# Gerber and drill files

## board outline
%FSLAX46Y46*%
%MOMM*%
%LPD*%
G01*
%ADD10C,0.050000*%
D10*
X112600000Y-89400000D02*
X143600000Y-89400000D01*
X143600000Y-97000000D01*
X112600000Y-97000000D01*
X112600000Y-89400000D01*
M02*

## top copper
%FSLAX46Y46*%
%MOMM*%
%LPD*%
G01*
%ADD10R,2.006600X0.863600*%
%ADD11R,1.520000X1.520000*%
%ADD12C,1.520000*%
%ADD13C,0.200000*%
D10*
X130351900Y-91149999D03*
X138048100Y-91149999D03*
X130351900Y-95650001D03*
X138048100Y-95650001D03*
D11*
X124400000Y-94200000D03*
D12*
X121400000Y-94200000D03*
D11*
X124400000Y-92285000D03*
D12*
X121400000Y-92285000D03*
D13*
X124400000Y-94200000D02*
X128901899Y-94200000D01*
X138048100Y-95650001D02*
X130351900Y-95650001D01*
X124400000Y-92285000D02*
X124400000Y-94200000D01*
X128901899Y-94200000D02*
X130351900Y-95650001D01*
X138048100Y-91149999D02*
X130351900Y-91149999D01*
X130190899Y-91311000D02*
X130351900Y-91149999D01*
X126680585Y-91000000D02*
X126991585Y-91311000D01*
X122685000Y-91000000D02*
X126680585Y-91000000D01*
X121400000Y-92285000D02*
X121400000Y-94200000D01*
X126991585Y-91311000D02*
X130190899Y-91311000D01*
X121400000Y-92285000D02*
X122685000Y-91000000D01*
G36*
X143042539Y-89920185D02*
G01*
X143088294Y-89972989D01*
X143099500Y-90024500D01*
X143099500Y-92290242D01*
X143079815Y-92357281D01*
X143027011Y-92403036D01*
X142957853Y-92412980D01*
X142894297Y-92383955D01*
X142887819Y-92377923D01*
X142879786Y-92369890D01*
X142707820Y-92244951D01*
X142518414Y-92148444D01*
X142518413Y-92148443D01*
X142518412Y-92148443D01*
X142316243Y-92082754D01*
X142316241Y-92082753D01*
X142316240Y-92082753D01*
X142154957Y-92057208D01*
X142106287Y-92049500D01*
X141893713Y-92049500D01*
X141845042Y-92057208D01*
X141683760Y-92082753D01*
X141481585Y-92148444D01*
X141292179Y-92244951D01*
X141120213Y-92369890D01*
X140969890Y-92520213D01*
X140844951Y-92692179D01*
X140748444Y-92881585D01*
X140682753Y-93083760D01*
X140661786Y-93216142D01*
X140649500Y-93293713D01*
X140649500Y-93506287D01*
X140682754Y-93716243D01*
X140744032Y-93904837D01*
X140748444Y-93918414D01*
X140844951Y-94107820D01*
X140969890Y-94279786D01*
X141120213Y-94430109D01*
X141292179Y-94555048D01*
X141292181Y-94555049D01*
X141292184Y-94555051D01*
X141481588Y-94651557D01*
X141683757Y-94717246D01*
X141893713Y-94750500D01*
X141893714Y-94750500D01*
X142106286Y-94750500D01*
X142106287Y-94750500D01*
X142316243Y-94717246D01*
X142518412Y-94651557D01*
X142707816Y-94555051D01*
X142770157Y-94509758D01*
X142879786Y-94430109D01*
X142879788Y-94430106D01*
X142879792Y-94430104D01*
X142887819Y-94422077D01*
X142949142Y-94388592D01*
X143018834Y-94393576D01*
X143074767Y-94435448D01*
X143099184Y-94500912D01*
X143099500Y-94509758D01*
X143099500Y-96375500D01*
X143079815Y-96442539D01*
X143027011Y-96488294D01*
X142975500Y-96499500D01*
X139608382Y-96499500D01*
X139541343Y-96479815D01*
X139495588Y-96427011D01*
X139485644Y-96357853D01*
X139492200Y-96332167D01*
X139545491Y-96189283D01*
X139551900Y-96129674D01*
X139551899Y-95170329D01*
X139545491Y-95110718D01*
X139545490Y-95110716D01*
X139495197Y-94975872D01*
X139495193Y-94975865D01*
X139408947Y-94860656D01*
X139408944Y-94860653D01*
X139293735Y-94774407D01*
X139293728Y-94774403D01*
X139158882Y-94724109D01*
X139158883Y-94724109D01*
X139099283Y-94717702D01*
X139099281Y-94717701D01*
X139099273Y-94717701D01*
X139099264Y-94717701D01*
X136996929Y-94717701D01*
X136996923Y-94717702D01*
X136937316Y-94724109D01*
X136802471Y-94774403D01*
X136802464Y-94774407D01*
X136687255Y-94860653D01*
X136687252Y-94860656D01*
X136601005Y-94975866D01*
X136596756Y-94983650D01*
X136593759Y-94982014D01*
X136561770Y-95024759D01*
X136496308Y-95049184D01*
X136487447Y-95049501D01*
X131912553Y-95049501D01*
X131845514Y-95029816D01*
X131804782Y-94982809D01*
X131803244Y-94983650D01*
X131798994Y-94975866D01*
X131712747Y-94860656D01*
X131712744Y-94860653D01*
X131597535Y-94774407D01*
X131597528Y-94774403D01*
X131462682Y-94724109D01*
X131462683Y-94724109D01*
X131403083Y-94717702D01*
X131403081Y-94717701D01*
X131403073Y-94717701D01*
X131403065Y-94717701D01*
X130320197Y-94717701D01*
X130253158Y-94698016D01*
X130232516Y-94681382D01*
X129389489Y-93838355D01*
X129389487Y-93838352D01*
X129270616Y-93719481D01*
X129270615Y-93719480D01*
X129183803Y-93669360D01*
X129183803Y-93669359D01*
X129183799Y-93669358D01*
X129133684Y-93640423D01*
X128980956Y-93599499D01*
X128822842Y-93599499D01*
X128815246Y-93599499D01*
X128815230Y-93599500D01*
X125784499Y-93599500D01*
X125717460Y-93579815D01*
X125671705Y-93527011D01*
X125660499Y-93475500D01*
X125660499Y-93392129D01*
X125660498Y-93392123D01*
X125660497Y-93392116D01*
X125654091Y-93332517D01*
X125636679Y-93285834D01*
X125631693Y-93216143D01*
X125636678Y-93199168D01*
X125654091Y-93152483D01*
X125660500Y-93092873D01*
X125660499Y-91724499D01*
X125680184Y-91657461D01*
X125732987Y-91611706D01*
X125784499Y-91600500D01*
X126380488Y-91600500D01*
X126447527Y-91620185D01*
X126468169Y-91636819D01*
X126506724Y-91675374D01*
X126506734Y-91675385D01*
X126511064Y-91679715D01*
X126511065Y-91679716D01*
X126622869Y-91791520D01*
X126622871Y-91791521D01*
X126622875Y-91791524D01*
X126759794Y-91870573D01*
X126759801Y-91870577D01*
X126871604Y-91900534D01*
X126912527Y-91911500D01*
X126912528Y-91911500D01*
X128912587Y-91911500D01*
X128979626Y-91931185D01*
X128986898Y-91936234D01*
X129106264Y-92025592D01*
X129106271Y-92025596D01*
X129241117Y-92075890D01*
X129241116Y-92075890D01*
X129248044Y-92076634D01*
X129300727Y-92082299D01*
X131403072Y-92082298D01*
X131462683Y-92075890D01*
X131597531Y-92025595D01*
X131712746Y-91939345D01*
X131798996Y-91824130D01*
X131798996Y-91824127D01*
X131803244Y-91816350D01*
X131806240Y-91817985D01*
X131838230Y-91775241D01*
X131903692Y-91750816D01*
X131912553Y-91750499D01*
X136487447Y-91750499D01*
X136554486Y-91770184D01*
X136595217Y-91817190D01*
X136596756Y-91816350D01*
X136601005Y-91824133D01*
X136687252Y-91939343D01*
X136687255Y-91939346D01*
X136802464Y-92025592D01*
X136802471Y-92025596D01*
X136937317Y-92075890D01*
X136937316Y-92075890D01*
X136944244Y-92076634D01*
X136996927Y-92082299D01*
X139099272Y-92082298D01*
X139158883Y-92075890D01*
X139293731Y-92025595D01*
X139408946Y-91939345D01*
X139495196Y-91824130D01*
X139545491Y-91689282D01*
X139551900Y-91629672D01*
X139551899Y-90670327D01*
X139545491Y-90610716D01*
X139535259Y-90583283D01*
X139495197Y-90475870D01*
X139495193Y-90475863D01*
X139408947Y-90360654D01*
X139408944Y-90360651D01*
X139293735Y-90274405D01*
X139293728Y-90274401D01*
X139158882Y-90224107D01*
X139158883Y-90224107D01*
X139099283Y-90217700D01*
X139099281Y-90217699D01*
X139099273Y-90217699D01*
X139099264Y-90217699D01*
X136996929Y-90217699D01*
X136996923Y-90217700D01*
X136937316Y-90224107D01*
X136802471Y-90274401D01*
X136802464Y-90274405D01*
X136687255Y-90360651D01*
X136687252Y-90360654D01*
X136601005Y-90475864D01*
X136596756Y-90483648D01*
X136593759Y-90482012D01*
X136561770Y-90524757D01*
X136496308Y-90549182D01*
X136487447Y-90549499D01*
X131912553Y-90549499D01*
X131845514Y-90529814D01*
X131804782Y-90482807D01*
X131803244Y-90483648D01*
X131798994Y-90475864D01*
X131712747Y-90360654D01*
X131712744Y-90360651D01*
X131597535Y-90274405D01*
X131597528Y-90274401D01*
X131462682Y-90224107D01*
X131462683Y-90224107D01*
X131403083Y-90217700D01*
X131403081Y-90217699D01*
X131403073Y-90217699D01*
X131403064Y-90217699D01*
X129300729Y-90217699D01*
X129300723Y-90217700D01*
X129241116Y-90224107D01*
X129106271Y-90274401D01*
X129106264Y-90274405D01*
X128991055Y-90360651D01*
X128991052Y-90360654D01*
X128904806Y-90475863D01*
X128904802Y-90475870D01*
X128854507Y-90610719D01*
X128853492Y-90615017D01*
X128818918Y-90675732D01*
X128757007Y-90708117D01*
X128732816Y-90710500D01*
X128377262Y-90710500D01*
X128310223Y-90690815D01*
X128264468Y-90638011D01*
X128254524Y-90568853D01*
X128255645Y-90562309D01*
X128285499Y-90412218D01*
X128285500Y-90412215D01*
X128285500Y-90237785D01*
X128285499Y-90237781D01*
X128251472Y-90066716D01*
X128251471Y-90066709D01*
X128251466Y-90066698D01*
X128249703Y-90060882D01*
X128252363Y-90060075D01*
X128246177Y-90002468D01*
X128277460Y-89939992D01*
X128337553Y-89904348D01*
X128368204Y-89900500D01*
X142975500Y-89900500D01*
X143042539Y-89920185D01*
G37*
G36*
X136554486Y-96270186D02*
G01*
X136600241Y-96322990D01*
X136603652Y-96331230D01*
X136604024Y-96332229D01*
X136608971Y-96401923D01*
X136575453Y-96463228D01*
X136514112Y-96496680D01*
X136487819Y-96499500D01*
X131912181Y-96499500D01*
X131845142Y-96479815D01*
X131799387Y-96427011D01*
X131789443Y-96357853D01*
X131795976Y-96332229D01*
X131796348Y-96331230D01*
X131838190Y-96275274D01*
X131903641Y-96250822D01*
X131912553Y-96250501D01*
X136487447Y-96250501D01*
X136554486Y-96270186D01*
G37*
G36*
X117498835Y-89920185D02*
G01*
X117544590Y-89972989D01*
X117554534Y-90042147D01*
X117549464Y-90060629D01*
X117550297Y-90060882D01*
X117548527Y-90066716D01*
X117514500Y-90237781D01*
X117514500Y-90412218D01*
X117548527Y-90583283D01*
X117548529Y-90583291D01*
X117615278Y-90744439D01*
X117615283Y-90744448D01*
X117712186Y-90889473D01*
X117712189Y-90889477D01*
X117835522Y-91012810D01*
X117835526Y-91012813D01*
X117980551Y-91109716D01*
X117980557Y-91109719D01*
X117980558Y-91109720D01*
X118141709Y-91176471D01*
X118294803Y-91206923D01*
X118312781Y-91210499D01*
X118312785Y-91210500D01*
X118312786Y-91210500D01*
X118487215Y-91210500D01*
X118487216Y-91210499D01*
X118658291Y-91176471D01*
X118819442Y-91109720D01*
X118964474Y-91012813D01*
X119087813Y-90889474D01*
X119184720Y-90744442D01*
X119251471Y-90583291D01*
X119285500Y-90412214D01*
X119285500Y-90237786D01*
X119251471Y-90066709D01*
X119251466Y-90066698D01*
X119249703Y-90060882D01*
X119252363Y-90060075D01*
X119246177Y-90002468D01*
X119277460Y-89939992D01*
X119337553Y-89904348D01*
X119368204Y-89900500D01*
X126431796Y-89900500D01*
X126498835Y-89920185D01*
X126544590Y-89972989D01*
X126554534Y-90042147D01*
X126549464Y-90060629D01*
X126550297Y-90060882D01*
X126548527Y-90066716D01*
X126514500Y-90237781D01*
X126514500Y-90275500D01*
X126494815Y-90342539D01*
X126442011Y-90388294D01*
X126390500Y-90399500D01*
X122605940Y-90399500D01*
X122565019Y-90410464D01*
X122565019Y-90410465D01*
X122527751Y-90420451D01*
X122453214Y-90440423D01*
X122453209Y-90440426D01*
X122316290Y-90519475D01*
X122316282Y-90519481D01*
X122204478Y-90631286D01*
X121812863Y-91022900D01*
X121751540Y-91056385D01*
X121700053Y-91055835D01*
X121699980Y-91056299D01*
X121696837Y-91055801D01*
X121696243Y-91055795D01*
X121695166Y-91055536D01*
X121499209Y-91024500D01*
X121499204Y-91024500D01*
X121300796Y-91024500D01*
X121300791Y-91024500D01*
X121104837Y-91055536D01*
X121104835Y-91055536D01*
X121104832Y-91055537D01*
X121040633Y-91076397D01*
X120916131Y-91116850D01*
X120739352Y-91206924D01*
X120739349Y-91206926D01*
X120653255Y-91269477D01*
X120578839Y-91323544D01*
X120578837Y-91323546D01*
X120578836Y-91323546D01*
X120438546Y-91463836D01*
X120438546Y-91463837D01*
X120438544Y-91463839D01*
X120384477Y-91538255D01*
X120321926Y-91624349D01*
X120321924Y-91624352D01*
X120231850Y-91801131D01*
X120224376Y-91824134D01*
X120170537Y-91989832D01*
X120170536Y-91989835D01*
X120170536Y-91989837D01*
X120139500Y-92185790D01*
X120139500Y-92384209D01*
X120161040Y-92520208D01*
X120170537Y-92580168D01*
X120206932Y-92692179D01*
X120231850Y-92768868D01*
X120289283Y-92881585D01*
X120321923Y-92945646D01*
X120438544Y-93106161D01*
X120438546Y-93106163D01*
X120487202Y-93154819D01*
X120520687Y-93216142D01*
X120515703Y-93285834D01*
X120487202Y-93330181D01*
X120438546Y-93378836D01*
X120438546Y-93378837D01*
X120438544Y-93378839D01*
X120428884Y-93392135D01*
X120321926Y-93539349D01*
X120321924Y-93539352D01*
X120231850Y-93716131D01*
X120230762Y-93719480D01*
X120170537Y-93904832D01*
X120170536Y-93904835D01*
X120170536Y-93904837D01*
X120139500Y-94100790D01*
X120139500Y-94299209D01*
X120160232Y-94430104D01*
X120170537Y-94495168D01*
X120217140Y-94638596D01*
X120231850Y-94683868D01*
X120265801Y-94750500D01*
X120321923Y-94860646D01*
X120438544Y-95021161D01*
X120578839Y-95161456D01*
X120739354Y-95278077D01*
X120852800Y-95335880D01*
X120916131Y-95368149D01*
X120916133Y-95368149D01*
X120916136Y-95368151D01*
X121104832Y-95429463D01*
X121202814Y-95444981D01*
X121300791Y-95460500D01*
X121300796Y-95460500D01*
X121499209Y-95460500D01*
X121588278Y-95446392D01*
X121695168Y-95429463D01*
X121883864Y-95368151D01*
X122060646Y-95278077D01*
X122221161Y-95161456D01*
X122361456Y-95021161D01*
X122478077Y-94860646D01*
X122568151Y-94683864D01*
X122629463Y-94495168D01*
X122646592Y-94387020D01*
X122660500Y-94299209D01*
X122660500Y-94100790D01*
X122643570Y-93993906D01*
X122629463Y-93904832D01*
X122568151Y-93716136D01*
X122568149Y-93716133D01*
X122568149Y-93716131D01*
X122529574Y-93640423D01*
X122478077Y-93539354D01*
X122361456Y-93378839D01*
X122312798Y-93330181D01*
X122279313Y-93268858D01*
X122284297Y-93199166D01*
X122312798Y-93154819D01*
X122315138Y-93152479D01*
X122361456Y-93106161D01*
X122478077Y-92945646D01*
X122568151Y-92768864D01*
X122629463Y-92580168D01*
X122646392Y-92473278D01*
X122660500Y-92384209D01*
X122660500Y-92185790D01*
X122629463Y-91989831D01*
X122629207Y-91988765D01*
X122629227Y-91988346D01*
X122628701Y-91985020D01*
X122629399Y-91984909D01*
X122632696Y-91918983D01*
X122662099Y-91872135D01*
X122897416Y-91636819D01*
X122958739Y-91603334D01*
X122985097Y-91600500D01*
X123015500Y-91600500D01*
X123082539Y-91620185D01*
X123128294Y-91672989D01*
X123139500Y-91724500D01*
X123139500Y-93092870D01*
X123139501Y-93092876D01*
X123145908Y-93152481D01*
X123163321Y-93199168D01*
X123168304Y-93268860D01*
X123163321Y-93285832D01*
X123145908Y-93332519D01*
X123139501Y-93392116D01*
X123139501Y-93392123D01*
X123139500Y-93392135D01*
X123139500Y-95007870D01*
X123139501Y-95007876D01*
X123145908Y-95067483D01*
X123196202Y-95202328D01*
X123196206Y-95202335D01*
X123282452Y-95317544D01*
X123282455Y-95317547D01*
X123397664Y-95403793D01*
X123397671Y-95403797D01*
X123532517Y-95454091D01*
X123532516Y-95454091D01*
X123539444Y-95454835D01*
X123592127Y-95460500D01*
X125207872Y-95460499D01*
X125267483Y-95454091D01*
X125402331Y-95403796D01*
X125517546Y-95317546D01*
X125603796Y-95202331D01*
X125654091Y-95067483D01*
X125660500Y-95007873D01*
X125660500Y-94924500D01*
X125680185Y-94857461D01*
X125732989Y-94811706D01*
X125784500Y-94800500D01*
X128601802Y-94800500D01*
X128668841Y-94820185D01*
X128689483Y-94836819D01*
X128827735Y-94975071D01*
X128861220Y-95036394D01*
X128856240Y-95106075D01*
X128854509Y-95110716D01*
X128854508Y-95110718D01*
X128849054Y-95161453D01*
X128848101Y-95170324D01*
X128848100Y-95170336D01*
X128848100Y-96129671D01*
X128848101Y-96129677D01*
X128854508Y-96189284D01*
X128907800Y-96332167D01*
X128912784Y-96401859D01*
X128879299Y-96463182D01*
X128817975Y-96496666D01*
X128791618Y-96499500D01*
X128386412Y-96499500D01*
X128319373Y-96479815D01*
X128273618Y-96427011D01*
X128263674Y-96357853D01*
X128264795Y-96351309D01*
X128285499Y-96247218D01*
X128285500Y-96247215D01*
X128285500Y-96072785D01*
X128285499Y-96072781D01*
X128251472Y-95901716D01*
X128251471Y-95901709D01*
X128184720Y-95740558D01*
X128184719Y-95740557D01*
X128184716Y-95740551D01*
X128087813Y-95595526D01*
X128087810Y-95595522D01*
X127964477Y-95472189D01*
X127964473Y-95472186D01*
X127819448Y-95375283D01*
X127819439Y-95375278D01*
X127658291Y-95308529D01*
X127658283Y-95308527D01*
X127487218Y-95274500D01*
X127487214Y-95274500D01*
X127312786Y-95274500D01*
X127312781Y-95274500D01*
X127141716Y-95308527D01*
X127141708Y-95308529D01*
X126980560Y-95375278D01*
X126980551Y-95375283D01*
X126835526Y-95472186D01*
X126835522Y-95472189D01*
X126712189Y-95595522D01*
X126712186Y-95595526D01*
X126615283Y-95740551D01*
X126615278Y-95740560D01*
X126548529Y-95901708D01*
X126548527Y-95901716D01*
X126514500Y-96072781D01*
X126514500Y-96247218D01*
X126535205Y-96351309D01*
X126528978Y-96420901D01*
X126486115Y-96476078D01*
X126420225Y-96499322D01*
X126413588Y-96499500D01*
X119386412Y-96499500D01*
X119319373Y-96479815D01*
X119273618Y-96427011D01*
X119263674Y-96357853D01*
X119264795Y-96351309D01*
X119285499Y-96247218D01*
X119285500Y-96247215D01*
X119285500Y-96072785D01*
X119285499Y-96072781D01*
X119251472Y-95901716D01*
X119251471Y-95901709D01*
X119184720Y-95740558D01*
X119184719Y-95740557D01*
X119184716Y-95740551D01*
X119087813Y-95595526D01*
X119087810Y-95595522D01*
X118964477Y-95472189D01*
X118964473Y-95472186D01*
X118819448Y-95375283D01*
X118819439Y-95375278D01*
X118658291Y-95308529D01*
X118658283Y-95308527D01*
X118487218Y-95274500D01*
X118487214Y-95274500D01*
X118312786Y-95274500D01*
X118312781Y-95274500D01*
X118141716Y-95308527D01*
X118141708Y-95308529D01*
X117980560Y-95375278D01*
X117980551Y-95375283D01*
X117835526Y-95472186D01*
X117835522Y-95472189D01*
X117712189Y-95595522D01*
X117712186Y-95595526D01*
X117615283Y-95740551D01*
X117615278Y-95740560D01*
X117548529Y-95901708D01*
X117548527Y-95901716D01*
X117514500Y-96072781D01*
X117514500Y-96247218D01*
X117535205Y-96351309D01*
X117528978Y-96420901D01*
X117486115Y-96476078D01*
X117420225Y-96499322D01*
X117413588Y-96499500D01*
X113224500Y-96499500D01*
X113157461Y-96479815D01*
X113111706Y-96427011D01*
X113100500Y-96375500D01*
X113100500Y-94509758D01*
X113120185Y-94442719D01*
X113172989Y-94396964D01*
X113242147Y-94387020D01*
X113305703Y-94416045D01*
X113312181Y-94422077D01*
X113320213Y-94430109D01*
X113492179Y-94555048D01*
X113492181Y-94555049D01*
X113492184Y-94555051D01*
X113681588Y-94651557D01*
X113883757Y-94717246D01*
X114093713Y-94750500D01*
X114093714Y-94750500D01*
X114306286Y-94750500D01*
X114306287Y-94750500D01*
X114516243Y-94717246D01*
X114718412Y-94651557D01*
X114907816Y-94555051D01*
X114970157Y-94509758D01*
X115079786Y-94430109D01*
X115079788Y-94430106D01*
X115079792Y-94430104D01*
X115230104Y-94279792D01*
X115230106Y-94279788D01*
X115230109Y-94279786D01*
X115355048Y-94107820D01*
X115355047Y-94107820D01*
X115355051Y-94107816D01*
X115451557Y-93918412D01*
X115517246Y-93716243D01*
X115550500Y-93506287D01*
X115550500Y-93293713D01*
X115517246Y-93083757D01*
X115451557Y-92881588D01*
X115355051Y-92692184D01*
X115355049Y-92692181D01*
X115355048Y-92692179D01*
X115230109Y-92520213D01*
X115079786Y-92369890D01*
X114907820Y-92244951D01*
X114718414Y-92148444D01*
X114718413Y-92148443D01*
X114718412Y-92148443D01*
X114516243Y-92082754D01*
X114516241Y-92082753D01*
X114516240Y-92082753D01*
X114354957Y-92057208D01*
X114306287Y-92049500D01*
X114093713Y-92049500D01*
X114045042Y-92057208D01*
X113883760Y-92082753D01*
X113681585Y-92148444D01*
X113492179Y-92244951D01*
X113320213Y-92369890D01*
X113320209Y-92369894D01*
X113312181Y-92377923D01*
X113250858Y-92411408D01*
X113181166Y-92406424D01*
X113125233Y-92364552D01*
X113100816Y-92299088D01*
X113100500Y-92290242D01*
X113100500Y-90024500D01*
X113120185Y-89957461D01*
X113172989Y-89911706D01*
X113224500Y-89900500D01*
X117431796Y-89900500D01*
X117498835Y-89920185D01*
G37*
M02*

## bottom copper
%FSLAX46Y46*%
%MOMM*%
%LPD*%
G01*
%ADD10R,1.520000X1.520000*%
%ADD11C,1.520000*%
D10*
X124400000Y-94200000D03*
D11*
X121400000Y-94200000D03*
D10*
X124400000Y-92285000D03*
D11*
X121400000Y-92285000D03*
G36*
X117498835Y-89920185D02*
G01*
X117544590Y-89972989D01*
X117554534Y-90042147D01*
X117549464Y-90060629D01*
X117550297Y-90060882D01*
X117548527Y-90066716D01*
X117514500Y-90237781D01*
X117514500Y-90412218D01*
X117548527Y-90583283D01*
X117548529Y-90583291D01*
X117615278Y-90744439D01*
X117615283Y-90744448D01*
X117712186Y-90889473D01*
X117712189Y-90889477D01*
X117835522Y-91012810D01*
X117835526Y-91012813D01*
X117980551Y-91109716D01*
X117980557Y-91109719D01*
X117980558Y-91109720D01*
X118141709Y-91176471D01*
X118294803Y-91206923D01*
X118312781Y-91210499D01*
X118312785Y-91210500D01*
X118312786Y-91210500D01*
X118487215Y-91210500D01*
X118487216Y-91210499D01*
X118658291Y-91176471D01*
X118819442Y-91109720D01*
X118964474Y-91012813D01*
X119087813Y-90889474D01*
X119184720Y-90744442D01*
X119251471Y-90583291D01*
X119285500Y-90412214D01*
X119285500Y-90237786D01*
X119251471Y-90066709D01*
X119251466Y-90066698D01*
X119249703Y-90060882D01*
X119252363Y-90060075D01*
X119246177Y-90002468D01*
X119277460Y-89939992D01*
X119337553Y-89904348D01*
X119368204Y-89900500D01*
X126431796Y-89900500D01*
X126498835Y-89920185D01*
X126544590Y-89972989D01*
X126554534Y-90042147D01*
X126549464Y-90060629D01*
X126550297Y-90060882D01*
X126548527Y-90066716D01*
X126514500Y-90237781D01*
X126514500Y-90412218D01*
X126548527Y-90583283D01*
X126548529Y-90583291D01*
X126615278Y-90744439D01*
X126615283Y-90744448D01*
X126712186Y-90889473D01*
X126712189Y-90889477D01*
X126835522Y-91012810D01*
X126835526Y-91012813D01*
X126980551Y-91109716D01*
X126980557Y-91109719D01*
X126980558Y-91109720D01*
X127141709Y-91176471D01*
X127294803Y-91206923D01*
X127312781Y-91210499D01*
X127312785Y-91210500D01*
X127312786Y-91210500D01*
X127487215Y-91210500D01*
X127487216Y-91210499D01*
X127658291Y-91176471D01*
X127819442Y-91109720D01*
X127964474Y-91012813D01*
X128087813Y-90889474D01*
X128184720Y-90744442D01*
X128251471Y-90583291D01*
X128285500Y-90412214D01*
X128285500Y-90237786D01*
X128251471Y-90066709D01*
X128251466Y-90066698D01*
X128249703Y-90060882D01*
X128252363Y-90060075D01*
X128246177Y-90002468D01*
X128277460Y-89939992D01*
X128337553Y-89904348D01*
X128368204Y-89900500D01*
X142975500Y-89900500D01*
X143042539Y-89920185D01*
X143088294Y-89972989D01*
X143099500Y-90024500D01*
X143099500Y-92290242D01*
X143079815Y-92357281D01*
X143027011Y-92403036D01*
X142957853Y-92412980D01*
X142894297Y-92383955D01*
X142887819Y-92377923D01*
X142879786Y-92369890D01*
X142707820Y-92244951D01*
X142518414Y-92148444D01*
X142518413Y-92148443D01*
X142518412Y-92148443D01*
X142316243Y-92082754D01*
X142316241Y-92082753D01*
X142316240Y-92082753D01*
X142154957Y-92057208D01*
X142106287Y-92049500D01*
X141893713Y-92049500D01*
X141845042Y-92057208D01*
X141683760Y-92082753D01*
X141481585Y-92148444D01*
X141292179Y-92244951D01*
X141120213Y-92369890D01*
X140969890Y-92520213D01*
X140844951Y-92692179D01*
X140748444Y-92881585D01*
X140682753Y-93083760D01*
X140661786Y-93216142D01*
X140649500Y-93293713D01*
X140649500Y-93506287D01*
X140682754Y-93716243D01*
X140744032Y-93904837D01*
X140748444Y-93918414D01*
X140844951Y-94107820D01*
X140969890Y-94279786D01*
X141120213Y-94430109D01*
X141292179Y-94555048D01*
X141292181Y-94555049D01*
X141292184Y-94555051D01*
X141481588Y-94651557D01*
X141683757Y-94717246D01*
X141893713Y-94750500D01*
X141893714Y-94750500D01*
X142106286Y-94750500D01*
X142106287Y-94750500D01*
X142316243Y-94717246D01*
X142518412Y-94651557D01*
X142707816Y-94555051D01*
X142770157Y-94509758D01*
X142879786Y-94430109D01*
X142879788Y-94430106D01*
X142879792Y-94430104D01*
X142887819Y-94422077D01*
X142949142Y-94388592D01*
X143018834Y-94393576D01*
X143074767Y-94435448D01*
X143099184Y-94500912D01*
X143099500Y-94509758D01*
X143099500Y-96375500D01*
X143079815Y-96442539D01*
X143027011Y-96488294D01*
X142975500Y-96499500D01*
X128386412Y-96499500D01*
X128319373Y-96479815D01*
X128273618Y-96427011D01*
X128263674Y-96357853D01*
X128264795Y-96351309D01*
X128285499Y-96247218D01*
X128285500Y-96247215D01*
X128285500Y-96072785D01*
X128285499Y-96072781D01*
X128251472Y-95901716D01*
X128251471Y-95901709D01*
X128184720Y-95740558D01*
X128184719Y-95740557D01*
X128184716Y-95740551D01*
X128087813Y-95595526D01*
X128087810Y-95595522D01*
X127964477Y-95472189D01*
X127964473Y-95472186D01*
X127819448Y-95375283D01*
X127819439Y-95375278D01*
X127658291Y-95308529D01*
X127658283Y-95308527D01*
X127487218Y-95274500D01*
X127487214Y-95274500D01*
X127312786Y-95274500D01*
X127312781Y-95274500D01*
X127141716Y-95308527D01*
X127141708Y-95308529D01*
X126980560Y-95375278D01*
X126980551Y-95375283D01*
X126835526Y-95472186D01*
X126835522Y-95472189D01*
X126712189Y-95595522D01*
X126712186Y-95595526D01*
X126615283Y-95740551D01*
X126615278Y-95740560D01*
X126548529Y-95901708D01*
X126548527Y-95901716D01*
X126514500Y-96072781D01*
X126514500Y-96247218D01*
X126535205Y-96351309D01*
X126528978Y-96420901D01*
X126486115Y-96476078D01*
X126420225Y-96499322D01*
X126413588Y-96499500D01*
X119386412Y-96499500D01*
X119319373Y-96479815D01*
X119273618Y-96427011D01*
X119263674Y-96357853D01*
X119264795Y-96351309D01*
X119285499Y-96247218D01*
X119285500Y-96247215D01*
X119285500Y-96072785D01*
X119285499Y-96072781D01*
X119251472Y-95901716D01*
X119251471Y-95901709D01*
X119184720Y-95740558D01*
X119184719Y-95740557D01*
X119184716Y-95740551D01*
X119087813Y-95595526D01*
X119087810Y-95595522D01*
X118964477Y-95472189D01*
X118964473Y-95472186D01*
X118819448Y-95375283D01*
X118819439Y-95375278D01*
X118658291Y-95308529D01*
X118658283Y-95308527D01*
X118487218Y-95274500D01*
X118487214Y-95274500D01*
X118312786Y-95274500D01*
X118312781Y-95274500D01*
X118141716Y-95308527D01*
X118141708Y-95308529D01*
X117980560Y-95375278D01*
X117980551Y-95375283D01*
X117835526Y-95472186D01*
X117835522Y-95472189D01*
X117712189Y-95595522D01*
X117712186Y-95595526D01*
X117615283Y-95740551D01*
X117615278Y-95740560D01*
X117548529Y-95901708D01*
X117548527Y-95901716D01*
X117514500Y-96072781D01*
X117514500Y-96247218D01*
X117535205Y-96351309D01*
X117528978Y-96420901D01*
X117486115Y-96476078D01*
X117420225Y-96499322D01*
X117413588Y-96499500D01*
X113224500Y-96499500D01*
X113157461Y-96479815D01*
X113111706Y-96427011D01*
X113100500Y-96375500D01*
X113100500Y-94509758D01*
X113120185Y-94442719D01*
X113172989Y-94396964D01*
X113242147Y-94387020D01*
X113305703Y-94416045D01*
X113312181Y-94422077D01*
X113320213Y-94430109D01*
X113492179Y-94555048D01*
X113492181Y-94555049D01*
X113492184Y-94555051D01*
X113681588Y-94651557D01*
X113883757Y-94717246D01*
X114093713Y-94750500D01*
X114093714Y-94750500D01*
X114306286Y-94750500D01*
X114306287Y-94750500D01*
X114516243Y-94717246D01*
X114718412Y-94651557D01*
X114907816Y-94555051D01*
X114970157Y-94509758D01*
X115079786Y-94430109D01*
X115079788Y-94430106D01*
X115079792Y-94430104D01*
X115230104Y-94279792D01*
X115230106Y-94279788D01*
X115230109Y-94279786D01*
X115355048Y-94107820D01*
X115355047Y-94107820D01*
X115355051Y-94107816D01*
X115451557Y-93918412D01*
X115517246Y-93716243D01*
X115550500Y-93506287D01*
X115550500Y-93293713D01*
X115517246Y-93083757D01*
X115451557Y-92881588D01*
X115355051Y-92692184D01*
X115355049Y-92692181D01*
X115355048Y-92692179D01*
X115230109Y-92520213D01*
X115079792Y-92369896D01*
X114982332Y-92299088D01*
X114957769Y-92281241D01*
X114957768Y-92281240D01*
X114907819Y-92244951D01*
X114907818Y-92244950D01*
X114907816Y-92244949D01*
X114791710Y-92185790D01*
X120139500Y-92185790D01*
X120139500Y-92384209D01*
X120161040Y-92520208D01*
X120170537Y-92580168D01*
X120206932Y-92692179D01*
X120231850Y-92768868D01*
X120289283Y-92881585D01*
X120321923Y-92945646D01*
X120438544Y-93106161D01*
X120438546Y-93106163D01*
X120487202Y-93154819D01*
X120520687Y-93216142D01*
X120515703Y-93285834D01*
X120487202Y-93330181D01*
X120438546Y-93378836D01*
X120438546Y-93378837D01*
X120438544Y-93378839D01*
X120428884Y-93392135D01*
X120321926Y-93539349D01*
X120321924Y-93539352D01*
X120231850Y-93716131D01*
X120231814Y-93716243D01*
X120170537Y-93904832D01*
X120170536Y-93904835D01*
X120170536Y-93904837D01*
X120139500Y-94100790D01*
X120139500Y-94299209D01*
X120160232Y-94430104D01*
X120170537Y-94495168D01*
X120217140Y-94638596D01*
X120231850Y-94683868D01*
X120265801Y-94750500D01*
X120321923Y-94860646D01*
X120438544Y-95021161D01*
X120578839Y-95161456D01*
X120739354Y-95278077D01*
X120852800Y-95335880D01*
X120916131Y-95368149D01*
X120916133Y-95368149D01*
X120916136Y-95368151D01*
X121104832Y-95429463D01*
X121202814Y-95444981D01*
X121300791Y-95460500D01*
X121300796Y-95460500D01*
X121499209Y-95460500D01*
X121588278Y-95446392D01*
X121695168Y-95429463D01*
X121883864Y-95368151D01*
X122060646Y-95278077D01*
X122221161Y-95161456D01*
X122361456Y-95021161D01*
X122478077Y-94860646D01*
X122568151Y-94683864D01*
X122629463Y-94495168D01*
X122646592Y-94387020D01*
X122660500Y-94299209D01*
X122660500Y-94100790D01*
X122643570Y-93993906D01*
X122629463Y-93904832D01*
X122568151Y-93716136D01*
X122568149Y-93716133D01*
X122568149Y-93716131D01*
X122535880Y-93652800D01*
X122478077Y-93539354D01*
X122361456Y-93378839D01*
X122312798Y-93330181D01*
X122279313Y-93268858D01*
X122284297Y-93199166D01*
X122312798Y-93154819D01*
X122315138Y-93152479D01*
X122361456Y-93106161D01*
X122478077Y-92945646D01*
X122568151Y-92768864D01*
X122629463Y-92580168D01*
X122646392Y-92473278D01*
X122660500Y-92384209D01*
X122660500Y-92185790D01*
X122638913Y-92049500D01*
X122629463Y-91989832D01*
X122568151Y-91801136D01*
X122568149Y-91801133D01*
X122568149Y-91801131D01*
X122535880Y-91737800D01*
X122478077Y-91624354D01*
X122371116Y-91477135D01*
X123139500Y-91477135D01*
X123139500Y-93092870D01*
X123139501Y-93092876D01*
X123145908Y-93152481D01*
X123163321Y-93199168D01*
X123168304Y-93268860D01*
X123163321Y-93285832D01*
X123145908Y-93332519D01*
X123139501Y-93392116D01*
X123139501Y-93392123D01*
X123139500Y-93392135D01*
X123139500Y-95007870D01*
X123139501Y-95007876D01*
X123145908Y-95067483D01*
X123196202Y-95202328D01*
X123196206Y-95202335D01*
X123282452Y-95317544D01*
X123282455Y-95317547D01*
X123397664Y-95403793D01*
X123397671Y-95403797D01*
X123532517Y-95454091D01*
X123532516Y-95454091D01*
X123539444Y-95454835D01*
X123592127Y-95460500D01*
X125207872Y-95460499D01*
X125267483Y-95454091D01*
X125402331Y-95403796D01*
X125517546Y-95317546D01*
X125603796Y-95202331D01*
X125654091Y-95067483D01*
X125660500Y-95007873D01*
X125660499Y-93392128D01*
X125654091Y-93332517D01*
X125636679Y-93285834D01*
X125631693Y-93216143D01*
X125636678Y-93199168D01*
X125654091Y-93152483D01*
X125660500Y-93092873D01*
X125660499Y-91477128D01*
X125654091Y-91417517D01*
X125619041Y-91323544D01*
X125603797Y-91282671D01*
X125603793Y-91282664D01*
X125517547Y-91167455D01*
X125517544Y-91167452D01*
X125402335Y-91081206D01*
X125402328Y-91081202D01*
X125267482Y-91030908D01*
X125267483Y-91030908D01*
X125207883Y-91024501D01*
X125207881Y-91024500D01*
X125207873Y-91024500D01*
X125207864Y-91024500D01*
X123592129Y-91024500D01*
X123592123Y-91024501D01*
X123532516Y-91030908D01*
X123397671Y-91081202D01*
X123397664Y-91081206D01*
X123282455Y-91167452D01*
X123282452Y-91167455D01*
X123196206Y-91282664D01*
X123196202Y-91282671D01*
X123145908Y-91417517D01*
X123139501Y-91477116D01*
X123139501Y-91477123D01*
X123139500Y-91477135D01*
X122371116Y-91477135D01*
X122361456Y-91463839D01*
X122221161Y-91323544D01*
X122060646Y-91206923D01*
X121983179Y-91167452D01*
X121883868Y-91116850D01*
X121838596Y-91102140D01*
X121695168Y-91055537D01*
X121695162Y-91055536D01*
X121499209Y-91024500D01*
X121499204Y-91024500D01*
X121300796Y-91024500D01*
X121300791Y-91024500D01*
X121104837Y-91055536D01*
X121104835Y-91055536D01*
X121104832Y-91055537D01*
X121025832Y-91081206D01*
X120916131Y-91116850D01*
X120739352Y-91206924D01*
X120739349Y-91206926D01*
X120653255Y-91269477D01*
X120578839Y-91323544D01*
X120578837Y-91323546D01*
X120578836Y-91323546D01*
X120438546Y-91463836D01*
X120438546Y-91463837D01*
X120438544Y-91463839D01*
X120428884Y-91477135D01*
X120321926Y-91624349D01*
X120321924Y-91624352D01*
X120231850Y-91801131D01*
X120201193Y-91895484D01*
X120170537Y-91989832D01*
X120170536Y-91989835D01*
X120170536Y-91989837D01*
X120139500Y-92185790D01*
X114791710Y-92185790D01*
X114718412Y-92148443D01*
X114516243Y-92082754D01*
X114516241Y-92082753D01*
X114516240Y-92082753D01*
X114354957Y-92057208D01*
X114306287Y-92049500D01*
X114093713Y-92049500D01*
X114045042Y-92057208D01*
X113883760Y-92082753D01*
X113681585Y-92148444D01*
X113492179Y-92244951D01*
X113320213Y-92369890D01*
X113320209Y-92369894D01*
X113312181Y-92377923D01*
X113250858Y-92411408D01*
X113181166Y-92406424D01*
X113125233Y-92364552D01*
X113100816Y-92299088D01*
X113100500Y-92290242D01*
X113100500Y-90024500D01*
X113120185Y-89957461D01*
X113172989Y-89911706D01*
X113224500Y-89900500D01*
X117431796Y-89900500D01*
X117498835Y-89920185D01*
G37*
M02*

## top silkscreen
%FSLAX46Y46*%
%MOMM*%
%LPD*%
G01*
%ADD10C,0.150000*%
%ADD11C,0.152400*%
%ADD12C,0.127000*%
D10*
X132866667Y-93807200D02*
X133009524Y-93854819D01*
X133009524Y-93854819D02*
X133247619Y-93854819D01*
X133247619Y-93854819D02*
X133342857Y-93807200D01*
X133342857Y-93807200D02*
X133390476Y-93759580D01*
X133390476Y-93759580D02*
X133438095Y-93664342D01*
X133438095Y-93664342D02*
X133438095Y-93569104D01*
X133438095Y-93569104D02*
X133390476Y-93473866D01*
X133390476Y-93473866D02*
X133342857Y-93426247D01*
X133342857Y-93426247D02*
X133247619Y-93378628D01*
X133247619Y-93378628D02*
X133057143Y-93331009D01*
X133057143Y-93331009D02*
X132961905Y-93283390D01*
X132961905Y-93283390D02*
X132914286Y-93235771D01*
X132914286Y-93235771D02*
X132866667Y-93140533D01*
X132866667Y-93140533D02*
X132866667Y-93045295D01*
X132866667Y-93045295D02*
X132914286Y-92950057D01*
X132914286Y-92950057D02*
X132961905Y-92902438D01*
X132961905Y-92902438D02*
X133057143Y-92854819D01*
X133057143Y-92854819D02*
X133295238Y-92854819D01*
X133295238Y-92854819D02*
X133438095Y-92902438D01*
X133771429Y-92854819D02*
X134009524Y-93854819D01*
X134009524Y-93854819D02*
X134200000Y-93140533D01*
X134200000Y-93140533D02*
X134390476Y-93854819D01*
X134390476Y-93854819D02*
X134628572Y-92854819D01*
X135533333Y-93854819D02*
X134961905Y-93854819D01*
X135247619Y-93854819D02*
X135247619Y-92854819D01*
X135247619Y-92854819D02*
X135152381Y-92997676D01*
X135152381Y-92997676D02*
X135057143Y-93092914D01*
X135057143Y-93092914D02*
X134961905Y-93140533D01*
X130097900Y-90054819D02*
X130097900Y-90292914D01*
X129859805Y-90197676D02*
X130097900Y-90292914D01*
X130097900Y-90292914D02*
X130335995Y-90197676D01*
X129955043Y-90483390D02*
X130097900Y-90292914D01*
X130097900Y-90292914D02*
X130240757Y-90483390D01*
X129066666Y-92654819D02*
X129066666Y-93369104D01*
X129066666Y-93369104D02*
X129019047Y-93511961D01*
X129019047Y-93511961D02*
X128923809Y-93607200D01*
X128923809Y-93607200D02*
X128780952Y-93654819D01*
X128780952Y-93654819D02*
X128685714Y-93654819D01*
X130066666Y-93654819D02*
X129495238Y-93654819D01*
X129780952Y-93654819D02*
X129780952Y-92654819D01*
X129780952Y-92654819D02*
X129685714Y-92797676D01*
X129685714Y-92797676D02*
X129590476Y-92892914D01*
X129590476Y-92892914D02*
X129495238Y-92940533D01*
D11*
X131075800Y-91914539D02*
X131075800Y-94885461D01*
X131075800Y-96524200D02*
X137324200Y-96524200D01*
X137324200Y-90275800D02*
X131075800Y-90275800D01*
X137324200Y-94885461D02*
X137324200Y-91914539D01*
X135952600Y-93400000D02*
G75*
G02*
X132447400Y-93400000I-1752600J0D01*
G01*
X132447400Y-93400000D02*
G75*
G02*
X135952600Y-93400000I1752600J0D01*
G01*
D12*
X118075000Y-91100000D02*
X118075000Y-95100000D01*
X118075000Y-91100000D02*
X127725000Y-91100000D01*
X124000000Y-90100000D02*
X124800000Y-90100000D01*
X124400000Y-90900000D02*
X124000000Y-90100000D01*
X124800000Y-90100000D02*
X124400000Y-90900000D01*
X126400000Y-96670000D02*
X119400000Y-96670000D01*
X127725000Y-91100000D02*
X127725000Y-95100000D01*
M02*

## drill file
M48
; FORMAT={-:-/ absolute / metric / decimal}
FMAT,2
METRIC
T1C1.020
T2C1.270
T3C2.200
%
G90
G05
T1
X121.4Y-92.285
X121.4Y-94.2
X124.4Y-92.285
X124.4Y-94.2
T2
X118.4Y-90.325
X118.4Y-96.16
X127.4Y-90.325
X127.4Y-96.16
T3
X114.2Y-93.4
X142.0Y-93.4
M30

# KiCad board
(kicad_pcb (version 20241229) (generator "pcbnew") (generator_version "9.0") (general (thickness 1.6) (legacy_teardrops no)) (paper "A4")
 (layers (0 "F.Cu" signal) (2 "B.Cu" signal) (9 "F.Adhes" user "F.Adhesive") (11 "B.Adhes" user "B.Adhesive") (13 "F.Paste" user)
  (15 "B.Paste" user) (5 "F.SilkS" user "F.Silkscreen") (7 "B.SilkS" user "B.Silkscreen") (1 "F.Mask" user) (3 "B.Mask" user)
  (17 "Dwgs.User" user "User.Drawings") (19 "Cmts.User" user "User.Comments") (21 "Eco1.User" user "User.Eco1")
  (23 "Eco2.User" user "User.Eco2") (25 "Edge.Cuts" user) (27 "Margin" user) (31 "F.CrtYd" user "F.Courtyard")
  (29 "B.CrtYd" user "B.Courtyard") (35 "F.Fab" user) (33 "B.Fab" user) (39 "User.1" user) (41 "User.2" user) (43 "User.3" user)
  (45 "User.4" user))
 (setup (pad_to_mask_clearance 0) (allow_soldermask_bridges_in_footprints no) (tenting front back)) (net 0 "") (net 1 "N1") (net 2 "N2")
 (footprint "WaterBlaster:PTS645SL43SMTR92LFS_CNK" (layer "F.Cu") (at 134.2 93.4)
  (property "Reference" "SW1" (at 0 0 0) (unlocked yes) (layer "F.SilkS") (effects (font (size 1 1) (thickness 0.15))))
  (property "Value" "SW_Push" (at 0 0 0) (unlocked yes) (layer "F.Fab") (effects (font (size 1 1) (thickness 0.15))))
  (fp_line (start -3.1242 -1.485461) (end -3.1242 1.485461) (stroke (width 0.1524) (type solid)) (layer "F.SilkS"))
  (fp_line (start -3.1242 3.1242) (end 3.1242 3.1242) (stroke (width 0.1524) (type solid)) (layer "F.SilkS"))
  (fp_line (start 3.1242 -3.1242) (end -3.1242 -3.1242) (stroke (width 0.1524) (type solid)) (layer "F.SilkS"))
  (fp_line (start 3.1242 1.485461) (end 3.1242 -1.485461) (stroke (width 0.1524) (type solid)) (layer "F.SilkS"))
  (fp_circle (center 0 0) (end 1.7526 0) (stroke (width 0.1524) (type solid)) (fill no) (layer "F.SilkS"))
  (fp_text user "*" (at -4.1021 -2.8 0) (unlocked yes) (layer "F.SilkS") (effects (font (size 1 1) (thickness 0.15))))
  (pad "1" smd rect (at -3.8481 -2.250001) (size 2.0066 0.8636) (layers "F.Cu" "F.Mask" "F.Paste") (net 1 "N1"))
  (pad "1" smd rect (at 3.8481 -2.250001) (size 2.0066 0.8636) (layers "F.Cu" "F.Mask" "F.Paste") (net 1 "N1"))
  (pad "2" smd rect (at -3.8481 2.250001) (size 2.0066 0.8636) (layers "F.Cu" "F.Mask" "F.Paste") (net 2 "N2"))
  (pad "2" smd rect (at 3.8481 2.250001) (size 2.0066 0.8636) (layers "F.Cu" "F.Mask" "F.Paste") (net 2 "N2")))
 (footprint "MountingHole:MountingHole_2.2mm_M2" (layer "F.Cu") (at 142 93.4)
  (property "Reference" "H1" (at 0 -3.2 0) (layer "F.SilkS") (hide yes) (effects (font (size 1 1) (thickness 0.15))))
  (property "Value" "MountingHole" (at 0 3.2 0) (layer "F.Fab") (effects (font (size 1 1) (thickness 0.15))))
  (pad "" np_thru_hole circle (at 0 0) (size 2.2 2.2) (drill 2.2) (layers "*.Cu" "*.Mask")))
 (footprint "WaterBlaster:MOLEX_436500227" (layer "F.Cu") (at 124.4 94.2)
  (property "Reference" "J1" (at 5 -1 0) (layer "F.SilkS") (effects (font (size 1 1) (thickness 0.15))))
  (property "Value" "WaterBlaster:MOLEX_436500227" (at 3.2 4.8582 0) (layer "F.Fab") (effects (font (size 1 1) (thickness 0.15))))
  (fp_line (start -6.325 -3.1) (end -6.325 0.9) (stroke (width 0.127) (type solid)) (layer "F.SilkS"))
  (fp_line (start -6.325 -3.1) (end 3.325 -3.1) (stroke (width 0.127) (type solid)) (layer "F.SilkS"))
  (fp_line (start -0.4 -4.1) (end 0.4 -4.1) (stroke (width 0.127) (type solid)) (layer "F.SilkS"))
  (fp_line (start 0 -3.3) (end -0.4 -4.1) (stroke (width 0.127) (type solid)) (layer "F.SilkS"))
  (fp_line (start 0.4 -4.1) (end 0 -3.3) (stroke (width 0.127) (type solid)) (layer "F.SilkS"))
  (fp_line (start 2 2.47) (end -5 2.47) (stroke (width 0.127) (type solid)) (layer "F.SilkS"))
  (fp_line (start 3.325 -3.1) (end 3.325 0.9) (stroke (width 0.127) (type solid)) (layer "F.SilkS"))
  (pad "" np_thru_hole circle (at -6 1.96) (size 1.27 1.27) (drill 1.27) (layers "*.Cu" "*.Mask"))
  (pad "" np_thru_hole circle (at 3 1.96) (size 1.27 1.27) (drill 1.27) (layers "*.Cu" "*.Mask"))
  (pad "1" thru_hole rect (at 0 0) (size 1.52 1.52) (drill 1.02) (layers "*.Cu") (remove_unused_layers no) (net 2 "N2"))
  (pad "2" thru_hole circle (at -3 0) (size 1.52 1.52) (drill 1.02) (layers "*.Cu") (remove_unused_layers no) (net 1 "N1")))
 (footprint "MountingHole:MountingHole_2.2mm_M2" (layer "F.Cu") (at 114.2 93.4)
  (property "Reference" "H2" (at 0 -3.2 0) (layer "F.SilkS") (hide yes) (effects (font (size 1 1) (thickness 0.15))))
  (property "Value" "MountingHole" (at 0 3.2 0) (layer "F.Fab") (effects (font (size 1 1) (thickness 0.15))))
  (pad "" np_thru_hole circle (at 0 0) (size 2.2 2.2) (drill 2.2) (layers "*.Cu" "*.Mask")))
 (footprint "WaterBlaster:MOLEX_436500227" (layer "B.Cu") (at 124.4 92.285)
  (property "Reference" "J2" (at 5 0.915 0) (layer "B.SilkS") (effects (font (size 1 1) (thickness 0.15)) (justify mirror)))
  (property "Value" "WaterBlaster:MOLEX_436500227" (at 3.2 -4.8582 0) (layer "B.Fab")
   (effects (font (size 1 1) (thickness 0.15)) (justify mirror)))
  (pad "" np_thru_hole circle (at -6 -1.96) (size 1.27 1.27) (drill 1.27) (layers "*.Cu" "*.Mask"))
  (pad "" np_thru_hole circle (at 3 -1.96) (size 1.27 1.27) (drill 1.27) (layers "*.Cu" "*.Mask"))
  (pad "1" thru_hole rect (at 0 0) (size 1.52 1.52) (drill 1.02) (layers "*.Cu") (remove_unused_layers no) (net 2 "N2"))
  (pad "2" thru_hole circle (at -3 0) (size 1.52 1.52) (drill 1.02) (layers "*.Cu") (remove_unused_layers no) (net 1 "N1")))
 (gr_rect (start 112.6 89.4) (end 143.6 97) (stroke (width 0.05) (type default)) (fill no) (layer "Edge.Cuts"))
 (segment (start 124.4 94.2) (end 128.901899 94.2) (width 0.2) (layer "F.Cu") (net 2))
 (segment (start 138.0481 95.650001) (end 130.3519 95.650001) (width 0.2) (layer "F.Cu") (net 2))
 (segment (start 124.4 92.285) (end 124.4 94.2) (width 0.2) (layer "F.Cu") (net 2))
 (segment (start 128.901899 94.2) (end 130.3519 95.650001) (width 0.2) (layer "F.Cu") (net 2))
 (segment (start 138.0481 91.149999) (end 130.3519 91.149999) (width 0.2) (layer "F.Cu") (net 1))
 (segment (start 130.190899 91.311) (end 130.3519 91.149999) (width 0.2) (layer "F.Cu") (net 1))
 (segment (start 126.680585 91) (end 126.991585 91.311) (width 0.2) (layer "F.Cu") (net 1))
 (segment (start 122.685 91) (end 126.680585 91) (width 0.2) (layer "F.Cu") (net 1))
 (segment (start 121.4 92.285) (end 121.4 94.2) (width 0.2) (layer "F.Cu") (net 1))
 (segment (start 126.991585 91.311) (end 130.190899 91.311) (width 0.2) (layer "F.Cu") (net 1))
 (segment (start 121.4 92.285) (end 122.685 91) (width 0.2) (layer "F.Cu") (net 1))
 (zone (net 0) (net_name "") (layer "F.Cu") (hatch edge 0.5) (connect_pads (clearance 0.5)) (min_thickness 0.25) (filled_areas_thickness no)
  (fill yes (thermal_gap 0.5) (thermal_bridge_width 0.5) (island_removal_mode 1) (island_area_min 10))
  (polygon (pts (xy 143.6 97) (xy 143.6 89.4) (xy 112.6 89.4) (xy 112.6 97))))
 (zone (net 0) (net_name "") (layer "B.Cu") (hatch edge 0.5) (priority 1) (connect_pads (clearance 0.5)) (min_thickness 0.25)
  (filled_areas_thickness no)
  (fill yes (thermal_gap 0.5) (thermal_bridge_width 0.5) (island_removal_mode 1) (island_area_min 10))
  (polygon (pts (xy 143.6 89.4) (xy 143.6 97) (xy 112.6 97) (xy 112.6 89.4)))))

